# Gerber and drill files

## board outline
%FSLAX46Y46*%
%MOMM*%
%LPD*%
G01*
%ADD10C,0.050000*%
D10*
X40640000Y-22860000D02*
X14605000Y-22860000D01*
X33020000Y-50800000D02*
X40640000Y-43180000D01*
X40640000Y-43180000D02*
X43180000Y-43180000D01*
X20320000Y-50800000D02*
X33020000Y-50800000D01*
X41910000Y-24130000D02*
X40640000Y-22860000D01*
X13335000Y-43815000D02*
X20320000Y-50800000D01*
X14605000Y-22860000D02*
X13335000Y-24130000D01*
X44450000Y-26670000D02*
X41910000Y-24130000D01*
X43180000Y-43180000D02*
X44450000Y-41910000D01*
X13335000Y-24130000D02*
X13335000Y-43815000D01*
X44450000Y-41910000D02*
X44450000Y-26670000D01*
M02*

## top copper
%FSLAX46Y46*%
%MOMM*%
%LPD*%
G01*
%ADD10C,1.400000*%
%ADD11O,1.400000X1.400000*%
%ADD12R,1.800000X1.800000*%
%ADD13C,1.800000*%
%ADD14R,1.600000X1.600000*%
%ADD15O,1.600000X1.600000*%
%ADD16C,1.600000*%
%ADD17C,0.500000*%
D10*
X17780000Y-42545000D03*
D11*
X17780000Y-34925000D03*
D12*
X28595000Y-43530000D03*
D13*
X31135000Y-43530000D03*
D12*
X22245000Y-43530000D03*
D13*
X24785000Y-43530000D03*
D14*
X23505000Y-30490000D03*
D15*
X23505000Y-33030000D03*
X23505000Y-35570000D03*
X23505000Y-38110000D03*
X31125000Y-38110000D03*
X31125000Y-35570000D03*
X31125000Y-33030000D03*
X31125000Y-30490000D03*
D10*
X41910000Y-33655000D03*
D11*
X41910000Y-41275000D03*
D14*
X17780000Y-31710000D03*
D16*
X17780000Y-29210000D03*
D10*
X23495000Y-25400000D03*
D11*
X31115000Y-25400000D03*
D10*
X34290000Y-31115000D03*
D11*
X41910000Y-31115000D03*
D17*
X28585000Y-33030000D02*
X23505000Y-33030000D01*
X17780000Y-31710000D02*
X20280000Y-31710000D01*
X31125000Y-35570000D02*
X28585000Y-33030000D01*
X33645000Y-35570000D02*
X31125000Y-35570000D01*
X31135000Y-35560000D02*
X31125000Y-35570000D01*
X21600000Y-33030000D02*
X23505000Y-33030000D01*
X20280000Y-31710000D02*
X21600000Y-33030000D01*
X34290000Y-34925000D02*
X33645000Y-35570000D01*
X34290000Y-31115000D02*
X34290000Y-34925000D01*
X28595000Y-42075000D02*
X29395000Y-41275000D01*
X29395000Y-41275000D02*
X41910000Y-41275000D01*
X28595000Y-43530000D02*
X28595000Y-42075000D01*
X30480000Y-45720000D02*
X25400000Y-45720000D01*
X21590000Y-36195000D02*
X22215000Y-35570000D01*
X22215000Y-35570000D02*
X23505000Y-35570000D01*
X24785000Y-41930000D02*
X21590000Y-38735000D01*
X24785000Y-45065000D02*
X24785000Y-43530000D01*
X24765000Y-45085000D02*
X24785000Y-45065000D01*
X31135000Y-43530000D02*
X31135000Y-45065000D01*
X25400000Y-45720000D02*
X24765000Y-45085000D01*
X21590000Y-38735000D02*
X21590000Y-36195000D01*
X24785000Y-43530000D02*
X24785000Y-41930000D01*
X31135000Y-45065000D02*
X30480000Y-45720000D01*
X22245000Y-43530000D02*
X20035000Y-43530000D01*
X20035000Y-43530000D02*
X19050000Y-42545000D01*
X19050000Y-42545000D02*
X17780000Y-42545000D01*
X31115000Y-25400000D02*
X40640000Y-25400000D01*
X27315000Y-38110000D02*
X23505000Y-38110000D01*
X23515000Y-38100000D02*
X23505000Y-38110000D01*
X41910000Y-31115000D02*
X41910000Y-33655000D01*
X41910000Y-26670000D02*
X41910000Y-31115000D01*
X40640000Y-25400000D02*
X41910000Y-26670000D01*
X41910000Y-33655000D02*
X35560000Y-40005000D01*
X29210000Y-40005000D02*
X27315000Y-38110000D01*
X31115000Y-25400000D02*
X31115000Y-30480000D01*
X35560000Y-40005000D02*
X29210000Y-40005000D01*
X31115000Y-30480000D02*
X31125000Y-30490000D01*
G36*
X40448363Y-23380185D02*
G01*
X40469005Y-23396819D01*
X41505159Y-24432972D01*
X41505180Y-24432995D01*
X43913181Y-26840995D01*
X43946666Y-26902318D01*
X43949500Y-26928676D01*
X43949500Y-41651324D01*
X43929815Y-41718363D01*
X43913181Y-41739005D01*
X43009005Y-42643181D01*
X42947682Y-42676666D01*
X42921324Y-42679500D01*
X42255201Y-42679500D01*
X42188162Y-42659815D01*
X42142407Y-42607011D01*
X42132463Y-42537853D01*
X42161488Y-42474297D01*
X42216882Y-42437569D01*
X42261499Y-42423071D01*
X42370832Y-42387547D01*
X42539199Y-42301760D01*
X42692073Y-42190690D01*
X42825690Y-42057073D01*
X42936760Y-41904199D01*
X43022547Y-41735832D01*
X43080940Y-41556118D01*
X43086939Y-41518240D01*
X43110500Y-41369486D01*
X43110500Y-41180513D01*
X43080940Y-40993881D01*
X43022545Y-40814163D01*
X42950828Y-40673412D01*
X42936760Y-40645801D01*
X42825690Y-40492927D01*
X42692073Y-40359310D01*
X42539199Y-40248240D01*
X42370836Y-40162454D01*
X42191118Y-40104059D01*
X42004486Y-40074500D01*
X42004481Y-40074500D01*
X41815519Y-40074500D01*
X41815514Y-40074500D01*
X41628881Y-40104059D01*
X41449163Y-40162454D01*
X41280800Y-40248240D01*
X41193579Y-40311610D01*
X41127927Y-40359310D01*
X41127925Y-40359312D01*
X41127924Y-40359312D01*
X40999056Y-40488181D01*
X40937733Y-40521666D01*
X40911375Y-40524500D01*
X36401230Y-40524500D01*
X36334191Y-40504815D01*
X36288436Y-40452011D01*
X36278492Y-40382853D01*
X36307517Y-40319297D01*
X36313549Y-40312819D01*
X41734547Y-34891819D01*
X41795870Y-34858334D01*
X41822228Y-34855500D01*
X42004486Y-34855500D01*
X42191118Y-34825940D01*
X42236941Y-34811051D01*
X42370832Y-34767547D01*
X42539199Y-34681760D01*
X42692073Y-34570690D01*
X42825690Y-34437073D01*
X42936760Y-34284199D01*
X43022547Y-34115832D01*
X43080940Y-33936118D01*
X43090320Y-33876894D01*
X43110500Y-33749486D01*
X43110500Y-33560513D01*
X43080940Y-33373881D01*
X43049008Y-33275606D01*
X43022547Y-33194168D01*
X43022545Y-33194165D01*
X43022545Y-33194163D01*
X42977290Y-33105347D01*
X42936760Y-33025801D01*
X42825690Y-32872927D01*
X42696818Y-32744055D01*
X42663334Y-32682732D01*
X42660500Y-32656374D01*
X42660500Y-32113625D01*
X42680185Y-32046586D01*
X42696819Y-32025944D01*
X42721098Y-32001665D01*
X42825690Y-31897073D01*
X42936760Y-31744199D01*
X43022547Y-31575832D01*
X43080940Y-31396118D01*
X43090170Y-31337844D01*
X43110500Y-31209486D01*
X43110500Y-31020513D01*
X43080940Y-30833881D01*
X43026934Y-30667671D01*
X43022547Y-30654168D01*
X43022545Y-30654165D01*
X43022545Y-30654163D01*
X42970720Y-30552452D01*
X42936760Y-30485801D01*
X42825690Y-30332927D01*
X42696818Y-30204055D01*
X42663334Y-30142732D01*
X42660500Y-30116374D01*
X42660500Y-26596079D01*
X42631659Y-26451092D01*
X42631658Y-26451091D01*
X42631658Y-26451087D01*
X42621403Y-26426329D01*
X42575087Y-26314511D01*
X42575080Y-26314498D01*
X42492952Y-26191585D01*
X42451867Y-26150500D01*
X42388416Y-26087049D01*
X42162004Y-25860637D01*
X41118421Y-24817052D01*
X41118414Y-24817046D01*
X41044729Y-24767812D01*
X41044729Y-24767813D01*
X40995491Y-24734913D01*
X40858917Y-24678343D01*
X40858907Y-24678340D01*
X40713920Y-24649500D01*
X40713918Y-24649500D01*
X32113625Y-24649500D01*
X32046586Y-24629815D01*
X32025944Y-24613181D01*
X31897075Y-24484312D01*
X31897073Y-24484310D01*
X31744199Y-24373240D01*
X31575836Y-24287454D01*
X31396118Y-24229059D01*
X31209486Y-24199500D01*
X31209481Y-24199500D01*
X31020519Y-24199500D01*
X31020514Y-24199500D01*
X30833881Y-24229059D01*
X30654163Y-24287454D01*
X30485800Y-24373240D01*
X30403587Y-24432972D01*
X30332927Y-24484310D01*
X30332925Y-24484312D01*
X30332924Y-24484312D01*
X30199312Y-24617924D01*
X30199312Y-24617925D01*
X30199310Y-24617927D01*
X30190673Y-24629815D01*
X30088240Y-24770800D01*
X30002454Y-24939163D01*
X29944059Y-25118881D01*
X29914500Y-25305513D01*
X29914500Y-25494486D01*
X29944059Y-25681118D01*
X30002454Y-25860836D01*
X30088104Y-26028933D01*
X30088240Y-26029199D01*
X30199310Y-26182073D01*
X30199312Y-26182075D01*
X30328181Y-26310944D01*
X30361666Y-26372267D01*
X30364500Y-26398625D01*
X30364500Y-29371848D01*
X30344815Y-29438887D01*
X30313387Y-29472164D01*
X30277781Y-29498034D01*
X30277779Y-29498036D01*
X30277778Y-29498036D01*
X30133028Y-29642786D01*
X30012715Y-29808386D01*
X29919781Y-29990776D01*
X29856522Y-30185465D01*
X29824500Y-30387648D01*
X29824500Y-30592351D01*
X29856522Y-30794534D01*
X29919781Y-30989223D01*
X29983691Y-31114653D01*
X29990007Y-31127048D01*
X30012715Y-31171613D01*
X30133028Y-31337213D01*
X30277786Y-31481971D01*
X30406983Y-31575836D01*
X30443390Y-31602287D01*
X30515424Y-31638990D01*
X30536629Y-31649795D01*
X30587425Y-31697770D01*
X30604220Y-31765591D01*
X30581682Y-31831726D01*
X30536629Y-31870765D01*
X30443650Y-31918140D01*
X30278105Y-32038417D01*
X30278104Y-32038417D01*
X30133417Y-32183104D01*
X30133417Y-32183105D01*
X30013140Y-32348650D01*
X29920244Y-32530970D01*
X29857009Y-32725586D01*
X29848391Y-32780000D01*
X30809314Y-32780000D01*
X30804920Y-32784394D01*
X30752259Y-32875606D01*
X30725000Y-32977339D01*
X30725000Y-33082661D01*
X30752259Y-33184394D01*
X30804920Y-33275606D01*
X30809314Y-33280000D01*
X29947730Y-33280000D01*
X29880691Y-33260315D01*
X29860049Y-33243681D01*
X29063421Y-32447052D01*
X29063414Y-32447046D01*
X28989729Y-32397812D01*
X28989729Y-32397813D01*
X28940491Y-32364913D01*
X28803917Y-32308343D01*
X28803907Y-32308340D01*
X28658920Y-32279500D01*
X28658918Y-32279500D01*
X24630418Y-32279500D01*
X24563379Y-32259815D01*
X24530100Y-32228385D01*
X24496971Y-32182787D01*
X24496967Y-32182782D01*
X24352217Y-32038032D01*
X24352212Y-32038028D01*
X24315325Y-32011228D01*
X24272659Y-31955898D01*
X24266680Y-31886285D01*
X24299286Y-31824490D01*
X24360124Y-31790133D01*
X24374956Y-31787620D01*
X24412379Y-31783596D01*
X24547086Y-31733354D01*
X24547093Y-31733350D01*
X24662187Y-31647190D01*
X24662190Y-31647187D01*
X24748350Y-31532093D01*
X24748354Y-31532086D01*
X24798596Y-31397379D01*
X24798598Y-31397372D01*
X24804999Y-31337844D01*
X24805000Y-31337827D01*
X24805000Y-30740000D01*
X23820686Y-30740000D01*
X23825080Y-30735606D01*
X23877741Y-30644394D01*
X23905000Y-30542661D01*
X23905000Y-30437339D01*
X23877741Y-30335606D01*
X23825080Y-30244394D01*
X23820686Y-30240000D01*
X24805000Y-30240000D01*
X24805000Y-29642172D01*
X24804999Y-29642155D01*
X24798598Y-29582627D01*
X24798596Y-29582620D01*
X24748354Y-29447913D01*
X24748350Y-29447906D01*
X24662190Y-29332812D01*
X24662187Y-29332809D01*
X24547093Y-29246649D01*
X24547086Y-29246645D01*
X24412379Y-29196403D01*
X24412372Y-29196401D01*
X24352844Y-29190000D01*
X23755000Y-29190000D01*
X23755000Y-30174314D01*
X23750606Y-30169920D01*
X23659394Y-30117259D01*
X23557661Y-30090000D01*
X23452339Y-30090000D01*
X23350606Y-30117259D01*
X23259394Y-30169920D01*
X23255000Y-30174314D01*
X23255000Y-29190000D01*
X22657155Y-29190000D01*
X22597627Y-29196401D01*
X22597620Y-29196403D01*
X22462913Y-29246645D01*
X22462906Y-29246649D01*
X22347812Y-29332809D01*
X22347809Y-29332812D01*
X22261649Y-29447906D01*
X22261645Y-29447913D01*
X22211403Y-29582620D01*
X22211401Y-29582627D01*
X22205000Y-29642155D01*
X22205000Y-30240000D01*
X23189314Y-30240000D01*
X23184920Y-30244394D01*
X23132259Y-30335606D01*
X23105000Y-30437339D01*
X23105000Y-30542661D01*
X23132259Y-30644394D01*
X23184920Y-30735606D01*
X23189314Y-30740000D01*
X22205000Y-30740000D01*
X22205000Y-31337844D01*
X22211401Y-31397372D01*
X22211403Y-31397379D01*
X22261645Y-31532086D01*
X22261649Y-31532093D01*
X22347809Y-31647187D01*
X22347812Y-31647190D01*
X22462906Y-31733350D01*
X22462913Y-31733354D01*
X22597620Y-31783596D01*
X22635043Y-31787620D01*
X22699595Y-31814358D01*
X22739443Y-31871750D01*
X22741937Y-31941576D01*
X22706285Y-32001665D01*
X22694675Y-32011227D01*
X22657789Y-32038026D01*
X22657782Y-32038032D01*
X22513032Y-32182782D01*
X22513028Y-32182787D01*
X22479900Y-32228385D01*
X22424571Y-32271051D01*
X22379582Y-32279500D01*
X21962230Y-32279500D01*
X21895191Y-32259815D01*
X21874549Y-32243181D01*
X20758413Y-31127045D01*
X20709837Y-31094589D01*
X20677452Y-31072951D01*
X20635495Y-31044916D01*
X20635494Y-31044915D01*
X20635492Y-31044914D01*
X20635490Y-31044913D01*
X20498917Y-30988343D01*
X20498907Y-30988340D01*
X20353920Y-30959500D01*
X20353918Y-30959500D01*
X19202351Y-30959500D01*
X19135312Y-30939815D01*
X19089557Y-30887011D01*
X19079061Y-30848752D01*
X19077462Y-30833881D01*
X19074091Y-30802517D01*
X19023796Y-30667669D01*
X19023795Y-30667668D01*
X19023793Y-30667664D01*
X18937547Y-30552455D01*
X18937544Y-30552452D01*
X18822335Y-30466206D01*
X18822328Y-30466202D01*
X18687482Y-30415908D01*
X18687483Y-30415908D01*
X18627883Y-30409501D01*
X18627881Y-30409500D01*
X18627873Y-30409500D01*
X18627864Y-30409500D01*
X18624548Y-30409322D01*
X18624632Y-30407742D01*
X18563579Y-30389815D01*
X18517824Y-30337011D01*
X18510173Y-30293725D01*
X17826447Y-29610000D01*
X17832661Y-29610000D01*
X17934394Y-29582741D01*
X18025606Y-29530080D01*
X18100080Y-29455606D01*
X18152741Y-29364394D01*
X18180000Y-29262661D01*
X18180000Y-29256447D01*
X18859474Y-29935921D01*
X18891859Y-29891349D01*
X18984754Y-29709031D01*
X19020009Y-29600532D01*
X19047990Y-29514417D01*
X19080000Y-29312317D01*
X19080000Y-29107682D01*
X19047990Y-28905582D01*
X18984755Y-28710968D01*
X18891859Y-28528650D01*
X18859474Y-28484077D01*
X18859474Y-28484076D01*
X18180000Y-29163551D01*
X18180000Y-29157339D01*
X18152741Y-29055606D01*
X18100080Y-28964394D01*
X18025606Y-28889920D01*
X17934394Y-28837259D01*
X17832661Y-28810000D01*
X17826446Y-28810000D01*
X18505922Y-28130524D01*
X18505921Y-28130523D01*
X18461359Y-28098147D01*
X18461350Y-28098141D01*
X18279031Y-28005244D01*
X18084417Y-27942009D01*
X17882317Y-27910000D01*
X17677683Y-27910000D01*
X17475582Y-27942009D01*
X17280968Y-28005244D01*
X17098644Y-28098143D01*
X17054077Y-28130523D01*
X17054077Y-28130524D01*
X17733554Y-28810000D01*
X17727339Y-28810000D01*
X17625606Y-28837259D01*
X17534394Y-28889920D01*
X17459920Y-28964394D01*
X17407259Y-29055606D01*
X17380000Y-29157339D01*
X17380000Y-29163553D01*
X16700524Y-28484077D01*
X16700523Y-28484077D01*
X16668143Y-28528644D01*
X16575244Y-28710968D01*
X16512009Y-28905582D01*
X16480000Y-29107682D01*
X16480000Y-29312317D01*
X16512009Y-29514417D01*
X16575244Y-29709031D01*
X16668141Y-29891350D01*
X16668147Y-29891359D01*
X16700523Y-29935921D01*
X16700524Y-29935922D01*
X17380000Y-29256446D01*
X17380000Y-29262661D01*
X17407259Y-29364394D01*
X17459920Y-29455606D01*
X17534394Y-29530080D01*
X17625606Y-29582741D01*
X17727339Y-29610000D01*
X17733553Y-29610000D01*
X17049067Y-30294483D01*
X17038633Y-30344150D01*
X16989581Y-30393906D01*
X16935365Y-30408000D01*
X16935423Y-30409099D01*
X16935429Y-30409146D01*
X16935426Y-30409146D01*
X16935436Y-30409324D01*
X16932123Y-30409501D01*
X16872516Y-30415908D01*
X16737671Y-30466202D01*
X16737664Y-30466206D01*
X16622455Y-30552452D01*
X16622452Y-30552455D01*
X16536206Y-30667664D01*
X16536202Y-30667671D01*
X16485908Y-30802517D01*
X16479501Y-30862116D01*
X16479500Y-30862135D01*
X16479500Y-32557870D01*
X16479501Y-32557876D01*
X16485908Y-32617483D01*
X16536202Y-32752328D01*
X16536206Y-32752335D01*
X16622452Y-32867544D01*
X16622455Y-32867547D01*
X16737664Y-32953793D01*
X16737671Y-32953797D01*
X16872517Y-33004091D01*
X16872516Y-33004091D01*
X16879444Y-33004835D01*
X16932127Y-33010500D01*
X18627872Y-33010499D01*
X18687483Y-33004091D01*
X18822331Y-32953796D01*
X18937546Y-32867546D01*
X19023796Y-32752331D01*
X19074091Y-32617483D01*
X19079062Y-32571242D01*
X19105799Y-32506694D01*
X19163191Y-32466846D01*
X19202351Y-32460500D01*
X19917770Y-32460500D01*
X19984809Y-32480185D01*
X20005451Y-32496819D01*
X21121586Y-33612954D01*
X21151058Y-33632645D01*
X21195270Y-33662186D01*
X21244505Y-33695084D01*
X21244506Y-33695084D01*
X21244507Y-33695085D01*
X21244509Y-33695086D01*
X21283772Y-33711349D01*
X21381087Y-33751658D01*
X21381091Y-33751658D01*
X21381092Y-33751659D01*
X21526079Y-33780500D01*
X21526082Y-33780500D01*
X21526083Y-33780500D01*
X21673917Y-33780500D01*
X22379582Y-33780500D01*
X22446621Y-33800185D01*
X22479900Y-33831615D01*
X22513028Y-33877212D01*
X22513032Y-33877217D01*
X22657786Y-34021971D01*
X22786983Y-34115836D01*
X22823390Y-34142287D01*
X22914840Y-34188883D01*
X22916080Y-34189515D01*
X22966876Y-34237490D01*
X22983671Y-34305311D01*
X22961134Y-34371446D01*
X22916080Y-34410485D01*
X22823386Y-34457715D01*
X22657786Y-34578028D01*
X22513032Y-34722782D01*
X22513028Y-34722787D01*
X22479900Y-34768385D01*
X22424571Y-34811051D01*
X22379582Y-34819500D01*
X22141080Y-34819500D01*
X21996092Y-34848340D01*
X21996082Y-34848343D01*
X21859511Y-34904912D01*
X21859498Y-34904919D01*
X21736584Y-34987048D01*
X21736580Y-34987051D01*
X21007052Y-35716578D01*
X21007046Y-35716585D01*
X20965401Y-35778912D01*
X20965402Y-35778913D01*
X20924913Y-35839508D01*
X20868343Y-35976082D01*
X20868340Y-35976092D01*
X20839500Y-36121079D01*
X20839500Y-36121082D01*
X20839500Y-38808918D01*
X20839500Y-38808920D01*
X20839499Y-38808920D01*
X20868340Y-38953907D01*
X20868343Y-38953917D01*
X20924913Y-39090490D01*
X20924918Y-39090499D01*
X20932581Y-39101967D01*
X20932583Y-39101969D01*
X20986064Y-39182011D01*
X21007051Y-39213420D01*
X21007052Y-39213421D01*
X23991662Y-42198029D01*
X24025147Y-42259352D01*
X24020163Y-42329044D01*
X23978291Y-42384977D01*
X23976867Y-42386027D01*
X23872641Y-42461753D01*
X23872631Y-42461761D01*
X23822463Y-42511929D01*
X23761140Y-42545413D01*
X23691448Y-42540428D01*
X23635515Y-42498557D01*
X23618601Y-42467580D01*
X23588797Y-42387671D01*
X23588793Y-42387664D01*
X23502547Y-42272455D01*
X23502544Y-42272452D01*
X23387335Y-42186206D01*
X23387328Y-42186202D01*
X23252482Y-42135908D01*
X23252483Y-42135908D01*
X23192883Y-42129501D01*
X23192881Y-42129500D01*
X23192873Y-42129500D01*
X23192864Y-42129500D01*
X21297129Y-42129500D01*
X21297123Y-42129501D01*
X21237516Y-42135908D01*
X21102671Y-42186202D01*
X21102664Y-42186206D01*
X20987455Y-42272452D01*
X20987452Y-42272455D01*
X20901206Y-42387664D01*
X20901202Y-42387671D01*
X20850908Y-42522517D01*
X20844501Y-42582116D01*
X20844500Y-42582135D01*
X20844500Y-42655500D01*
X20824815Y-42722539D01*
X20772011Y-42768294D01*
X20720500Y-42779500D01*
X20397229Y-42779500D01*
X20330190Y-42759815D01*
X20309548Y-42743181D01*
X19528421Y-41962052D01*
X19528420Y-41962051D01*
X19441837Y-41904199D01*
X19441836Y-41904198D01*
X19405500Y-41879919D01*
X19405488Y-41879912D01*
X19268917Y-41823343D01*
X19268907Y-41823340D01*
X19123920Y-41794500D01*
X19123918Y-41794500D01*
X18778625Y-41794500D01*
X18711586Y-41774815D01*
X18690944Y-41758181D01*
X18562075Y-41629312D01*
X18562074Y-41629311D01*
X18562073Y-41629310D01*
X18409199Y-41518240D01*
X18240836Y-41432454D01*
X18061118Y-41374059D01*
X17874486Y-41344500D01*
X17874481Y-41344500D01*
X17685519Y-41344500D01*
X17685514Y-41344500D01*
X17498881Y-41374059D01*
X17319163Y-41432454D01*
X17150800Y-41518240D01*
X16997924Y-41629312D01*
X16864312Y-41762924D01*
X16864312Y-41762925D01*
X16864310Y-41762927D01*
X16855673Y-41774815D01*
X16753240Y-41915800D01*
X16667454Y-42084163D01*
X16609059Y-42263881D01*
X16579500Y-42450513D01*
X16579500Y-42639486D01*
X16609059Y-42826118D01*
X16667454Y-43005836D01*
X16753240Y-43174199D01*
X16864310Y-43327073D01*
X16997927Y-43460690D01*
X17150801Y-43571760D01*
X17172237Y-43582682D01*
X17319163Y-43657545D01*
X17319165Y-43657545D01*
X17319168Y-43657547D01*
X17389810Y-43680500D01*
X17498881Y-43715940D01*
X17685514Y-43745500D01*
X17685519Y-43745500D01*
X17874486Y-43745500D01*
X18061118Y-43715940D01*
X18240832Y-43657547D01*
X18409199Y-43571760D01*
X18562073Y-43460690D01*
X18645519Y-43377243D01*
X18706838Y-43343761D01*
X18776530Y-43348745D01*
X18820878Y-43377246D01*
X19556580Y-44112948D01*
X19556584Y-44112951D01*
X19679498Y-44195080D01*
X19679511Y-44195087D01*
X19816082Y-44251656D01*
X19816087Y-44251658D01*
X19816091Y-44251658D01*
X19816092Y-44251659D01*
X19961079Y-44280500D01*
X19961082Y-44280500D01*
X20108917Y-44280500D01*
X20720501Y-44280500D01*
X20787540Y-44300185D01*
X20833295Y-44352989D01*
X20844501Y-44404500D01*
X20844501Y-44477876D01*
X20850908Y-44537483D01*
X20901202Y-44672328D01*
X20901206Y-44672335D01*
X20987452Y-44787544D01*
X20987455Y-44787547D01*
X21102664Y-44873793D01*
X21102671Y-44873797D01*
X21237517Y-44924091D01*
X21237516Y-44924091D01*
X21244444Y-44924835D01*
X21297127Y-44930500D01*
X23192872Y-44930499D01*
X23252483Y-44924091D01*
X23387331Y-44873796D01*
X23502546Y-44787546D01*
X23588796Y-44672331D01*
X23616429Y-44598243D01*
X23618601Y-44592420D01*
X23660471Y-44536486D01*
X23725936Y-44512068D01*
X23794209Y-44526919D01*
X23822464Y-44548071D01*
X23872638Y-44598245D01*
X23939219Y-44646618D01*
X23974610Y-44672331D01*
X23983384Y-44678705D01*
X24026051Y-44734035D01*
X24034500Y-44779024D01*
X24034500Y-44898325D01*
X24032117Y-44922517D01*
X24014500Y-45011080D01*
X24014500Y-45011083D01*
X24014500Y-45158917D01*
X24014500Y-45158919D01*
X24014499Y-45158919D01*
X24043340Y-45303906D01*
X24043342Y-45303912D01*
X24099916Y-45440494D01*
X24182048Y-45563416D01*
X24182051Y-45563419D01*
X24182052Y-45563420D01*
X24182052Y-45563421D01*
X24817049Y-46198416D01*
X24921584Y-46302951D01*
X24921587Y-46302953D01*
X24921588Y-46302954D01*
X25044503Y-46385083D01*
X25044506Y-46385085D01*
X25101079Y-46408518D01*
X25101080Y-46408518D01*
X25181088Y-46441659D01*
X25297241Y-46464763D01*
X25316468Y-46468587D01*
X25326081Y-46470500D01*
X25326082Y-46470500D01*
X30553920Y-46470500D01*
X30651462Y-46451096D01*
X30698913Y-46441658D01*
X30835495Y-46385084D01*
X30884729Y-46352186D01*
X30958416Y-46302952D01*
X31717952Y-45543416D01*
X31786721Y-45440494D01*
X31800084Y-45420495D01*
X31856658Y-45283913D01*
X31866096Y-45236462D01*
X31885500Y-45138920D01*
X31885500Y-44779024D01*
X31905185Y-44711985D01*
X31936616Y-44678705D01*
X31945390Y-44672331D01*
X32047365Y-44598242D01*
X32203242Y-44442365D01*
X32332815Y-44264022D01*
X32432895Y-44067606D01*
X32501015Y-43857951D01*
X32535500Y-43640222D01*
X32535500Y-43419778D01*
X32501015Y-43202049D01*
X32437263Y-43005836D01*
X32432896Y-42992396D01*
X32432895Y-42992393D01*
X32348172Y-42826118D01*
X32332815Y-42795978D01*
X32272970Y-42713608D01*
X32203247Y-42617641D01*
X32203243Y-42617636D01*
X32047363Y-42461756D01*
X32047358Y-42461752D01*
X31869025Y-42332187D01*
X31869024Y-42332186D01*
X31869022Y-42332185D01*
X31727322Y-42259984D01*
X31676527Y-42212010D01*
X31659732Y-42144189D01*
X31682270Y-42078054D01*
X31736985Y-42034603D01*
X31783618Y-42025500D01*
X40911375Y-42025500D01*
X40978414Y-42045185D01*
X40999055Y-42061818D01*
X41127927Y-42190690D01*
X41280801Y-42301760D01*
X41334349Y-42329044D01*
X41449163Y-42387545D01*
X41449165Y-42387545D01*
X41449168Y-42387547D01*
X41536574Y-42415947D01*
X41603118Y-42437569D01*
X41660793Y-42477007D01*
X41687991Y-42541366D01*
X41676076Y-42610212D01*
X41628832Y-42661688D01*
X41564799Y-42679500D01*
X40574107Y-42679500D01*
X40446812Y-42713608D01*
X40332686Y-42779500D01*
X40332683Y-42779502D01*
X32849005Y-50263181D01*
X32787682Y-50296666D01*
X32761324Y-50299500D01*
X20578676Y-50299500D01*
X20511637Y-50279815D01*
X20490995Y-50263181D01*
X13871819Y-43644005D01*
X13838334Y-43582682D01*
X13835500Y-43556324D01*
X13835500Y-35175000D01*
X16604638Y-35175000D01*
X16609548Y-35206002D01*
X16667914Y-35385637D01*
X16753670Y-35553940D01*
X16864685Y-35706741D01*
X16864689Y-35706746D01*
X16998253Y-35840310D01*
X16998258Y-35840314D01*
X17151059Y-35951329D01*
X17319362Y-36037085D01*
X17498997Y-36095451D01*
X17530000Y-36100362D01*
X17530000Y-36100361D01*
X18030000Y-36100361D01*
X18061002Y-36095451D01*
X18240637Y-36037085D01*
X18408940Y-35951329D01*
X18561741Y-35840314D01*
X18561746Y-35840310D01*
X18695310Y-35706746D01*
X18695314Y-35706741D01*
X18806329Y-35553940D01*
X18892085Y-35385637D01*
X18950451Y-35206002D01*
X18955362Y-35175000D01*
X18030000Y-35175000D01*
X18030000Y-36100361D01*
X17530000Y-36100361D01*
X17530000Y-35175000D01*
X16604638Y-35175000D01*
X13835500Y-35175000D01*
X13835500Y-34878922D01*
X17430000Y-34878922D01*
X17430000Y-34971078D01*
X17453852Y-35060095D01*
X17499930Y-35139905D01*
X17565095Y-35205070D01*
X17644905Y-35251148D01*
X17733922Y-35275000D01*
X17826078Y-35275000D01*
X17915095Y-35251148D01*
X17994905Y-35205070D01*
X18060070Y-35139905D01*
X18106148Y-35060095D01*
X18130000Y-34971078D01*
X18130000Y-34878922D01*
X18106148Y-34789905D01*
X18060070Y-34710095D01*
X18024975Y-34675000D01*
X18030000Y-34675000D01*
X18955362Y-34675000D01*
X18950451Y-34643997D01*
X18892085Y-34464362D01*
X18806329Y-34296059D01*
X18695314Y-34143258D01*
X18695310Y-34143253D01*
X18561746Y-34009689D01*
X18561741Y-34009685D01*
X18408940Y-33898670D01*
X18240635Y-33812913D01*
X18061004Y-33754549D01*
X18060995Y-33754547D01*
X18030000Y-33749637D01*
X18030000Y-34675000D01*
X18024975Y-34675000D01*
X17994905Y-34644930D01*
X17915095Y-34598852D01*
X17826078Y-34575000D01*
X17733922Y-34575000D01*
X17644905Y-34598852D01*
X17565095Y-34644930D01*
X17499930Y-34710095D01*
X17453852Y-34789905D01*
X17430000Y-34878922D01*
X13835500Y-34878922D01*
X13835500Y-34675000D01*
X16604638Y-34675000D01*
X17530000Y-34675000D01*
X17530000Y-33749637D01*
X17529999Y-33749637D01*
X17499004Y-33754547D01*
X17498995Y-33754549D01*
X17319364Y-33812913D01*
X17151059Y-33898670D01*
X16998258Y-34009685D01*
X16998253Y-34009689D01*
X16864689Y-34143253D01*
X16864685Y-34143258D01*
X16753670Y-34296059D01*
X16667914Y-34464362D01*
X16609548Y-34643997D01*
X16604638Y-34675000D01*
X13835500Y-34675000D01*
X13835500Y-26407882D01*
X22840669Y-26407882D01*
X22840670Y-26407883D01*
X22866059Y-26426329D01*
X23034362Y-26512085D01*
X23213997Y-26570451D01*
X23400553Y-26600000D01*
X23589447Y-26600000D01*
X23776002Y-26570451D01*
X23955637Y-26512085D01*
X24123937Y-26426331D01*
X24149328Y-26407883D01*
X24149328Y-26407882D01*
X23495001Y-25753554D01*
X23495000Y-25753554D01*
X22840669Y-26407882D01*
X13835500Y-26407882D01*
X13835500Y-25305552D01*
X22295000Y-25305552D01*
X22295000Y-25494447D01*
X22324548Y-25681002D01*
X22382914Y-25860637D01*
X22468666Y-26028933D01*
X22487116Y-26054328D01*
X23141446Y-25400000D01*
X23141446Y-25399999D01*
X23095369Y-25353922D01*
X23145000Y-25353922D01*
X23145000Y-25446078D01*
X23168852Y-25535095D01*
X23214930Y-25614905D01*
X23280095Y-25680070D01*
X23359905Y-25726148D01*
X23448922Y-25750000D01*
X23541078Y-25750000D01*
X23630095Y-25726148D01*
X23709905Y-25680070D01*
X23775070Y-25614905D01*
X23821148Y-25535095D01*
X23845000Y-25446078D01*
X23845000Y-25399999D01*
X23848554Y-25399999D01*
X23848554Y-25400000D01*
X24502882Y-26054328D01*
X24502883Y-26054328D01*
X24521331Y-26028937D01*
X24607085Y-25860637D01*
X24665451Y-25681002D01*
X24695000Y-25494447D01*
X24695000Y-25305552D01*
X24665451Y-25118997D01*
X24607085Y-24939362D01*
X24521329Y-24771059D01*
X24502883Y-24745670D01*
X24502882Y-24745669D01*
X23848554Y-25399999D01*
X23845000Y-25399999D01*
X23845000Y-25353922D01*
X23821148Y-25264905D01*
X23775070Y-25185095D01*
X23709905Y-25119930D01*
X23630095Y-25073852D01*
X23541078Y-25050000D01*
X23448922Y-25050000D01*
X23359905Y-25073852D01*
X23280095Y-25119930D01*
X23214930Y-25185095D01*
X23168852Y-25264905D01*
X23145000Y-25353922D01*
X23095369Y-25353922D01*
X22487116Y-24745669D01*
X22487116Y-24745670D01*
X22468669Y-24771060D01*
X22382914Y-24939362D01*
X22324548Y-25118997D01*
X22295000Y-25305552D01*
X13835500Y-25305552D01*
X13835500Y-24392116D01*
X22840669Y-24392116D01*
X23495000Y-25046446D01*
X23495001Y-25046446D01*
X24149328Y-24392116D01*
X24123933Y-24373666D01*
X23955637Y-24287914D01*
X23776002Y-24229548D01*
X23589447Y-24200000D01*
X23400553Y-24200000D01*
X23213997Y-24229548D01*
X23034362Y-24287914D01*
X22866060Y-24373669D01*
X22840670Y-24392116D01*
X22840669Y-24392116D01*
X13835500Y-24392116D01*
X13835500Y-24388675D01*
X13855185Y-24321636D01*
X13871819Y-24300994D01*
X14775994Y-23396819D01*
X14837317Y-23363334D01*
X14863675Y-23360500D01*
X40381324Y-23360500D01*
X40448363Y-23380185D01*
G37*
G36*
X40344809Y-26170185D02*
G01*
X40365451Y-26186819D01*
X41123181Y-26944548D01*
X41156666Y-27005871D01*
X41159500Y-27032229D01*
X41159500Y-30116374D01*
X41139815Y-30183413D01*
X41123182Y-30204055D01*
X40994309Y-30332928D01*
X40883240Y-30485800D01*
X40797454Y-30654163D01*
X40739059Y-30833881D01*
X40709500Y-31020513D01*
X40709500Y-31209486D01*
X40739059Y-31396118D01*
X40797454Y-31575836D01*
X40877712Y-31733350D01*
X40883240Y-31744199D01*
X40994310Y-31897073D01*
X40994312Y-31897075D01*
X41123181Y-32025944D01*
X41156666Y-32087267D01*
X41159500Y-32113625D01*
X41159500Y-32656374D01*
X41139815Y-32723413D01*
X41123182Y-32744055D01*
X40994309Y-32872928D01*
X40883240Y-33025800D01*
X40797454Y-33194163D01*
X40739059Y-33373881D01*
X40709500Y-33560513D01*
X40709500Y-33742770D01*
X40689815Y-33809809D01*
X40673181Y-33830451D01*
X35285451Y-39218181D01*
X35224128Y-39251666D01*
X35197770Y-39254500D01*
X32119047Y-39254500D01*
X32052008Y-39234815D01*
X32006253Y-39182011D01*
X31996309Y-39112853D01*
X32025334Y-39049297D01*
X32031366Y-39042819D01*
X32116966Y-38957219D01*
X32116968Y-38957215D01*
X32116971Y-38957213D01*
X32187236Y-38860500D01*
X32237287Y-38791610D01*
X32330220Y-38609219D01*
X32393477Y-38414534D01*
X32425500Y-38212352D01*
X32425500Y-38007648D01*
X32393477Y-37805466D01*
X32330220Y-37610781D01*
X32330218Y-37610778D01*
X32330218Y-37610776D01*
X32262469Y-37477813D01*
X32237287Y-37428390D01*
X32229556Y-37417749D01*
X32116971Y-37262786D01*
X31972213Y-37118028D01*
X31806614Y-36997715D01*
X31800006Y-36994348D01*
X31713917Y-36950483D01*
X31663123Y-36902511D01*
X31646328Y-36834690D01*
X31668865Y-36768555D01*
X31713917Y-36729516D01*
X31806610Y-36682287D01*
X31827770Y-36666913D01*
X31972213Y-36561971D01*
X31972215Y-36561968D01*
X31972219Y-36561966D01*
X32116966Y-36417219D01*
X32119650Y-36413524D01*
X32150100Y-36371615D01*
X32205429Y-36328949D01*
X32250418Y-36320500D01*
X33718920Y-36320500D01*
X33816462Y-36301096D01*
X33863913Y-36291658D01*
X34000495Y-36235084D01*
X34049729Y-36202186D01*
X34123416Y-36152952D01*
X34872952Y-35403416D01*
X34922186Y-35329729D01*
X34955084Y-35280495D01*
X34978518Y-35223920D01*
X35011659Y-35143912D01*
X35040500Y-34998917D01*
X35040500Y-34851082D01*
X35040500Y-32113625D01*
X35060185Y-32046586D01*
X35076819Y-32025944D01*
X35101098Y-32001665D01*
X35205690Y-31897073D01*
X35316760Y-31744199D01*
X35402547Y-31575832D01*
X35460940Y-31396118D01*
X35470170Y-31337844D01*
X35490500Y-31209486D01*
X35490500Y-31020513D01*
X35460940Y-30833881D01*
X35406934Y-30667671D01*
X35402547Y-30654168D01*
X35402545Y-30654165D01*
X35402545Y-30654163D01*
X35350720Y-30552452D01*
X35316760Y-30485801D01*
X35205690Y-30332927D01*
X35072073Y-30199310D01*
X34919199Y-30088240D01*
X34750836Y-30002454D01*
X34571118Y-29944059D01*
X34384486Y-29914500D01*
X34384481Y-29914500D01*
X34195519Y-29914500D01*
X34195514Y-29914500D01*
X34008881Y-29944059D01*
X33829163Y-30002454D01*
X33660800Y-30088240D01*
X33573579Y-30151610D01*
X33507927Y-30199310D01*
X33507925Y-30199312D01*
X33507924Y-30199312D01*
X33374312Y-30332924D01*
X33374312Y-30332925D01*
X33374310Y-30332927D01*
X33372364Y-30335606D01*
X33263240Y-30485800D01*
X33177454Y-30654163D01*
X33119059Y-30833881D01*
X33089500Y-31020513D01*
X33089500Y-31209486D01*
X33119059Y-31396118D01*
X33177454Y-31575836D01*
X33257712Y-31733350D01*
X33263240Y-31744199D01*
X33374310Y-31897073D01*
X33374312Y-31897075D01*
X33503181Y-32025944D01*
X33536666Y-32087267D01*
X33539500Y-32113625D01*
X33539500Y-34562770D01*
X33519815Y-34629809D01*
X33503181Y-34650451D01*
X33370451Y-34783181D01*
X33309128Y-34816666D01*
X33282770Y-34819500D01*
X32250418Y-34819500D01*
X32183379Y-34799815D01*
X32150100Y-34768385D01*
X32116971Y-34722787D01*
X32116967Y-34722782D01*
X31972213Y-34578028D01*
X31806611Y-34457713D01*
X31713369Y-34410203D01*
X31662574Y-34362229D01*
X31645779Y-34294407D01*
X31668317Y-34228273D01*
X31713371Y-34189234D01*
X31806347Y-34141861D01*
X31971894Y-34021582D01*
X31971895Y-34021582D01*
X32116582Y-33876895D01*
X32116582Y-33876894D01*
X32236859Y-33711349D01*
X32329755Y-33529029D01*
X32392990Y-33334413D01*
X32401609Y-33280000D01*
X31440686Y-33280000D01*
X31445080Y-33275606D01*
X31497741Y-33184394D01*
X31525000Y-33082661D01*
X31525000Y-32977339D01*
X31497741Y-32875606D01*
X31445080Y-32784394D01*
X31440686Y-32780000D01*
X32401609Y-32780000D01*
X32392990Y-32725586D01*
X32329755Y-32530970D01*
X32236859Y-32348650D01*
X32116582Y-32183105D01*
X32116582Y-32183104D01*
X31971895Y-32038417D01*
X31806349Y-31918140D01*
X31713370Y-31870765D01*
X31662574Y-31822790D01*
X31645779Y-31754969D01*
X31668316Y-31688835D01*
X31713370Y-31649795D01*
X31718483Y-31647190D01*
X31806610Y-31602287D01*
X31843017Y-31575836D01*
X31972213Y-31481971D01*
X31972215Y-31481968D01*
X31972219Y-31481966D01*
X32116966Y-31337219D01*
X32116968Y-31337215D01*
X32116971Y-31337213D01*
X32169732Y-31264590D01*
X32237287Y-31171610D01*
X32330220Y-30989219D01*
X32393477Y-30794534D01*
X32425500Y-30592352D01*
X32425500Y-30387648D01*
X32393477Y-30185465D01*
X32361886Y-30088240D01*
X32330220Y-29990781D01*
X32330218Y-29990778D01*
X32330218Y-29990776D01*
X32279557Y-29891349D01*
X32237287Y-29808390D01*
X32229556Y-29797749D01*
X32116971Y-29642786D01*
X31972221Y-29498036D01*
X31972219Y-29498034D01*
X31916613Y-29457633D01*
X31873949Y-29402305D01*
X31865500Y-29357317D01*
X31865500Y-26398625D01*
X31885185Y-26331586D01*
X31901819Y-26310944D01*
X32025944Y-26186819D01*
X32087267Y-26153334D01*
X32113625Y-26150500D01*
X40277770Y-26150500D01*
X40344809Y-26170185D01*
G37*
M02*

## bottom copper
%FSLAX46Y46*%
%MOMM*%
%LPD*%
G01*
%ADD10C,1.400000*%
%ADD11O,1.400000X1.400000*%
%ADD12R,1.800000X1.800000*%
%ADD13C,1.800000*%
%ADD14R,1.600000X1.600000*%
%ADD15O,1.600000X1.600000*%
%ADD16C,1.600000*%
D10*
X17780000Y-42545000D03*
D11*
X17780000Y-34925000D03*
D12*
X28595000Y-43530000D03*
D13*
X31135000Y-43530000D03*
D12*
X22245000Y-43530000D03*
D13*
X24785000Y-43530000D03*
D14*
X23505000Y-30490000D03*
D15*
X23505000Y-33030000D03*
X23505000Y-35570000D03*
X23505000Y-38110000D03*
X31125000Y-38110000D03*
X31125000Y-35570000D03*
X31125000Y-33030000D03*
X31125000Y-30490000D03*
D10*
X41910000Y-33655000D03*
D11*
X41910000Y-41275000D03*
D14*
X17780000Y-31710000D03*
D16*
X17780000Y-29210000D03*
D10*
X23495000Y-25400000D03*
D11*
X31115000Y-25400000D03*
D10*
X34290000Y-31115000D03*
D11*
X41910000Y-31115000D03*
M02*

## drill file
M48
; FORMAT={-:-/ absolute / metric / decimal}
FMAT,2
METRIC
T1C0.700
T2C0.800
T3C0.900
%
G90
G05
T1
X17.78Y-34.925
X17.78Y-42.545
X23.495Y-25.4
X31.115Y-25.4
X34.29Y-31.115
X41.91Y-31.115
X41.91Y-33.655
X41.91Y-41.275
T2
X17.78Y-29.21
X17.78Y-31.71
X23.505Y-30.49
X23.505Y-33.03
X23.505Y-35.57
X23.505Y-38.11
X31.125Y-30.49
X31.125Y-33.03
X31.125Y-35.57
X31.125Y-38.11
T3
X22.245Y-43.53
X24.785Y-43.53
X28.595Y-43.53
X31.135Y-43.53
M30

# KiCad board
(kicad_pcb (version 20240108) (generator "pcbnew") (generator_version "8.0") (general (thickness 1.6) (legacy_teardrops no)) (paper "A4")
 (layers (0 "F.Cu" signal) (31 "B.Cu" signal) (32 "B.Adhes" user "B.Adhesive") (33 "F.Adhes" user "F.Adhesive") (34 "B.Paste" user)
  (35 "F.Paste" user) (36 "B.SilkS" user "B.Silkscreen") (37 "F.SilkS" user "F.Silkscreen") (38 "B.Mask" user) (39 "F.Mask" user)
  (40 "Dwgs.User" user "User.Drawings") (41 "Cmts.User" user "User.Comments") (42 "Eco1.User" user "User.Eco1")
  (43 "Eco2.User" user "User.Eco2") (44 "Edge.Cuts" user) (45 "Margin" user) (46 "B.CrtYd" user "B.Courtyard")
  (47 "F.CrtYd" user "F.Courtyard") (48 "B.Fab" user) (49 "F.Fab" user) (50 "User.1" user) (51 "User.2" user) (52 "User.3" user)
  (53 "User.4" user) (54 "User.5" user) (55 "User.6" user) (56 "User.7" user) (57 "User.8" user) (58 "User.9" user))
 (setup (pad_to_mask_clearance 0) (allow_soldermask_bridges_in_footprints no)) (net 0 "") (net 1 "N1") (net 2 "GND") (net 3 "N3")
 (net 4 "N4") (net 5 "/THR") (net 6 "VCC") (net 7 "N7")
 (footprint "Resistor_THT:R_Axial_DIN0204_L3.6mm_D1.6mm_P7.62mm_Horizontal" (layer "F.Cu") (at 17.78 42.545 90)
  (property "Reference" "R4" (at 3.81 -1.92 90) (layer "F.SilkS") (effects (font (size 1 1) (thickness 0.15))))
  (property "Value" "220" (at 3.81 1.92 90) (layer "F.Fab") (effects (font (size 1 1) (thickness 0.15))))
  (pad "1" thru_hole circle (at 0 0 90) (size 1.4 1.4) (drill 0.7) (layers "*.Cu" "*.Mask") (remove_unused_layers no) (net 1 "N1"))
  (pad "2" thru_hole oval (at 7.62 0 90) (size 1.4 1.4) (drill 0.7) (layers "*.Cu" "*.Mask") (remove_unused_layers no) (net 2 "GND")))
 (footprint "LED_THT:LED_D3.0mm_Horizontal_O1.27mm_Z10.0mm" (layer "F.Cu") (at 28.595 43.53)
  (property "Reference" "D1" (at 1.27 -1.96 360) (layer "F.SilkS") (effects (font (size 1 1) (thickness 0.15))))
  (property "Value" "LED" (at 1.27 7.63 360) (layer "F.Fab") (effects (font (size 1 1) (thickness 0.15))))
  (pad "1" thru_hole rect (at 0 0) (size 1.8 1.8) (drill 0.9) (layers "*.Cu" "*.Mask") (remove_unused_layers no) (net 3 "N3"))
  (pad "2" thru_hole circle (at 2.54 0) (size 1.8 1.8) (drill 0.9) (layers "*.Cu" "*.Mask") (remove_unused_layers no) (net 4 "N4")))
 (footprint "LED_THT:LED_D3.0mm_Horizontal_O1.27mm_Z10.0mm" (layer "F.Cu") (at 22.245 43.53)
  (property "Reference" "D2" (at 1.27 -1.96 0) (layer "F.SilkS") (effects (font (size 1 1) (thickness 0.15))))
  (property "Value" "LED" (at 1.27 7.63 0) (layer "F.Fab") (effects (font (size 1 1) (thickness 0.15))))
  (pad "1" thru_hole rect (at 0 0) (size 1.8 1.8) (drill 0.9) (layers "*.Cu" "*.Mask") (remove_unused_layers no) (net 1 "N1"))
  (pad "2" thru_hole circle (at 2.54 0) (size 1.8 1.8) (drill 0.9) (layers "*.Cu" "*.Mask") (remove_unused_layers no) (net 4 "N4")))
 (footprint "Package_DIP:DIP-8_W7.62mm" (layer "F.Cu") (at 23.505 30.49)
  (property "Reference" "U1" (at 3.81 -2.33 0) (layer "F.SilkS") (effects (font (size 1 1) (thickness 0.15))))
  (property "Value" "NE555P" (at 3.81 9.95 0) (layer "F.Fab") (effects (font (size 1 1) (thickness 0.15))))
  (pad "1" thru_hole rect (at 0 0) (size 1.6 1.6) (drill 0.8) (layers "*.Cu" "*.Mask") (remove_unused_layers no) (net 2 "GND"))
  (pad "2" thru_hole oval (at 0 2.54) (size 1.6 1.6) (drill 0.8) (layers "*.Cu" "*.Mask") (remove_unused_layers no) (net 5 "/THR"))
  (pad "3" thru_hole oval (at 0 5.08) (size 1.6 1.6) (drill 0.8) (layers "*.Cu" "*.Mask") (remove_unused_layers no) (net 4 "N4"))
  (pad "4" thru_hole oval (at 0 7.62) (size 1.6 1.6) (drill 0.8) (layers "*.Cu" "*.Mask") (remove_unused_layers no) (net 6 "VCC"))
  (pad "5" thru_hole oval (at 7.62 7.62) (size 1.6 1.6) (drill 0.8) (layers "*.Cu" "*.Mask") (remove_unused_layers no) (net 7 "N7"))
  (pad "6" thru_hole oval (at 7.62 5.08) (size 1.6 1.6) (drill 0.8) (layers "*.Cu" "*.Mask") (remove_unused_layers no) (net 5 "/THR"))
  (pad "7" thru_hole oval (at 7.62 2.54) (size 1.6 1.6) (drill 0.8) (layers "*.Cu" "*.Mask") (remove_unused_layers no) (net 2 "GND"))
  (pad "8" thru_hole oval (at 7.62 0) (size 1.6 1.6) (drill 0.8) (layers "*.Cu" "*.Mask") (remove_unused_layers no) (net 6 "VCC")))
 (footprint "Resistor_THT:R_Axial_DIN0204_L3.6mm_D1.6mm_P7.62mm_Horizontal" (layer "F.Cu") (at 41.91 33.655 -90)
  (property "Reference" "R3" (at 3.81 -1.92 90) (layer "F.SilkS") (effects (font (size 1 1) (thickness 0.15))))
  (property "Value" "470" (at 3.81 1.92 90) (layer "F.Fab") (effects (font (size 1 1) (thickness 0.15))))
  (pad "1" thru_hole circle (at 0 0 270) (size 1.4 1.4) (drill 0.7) (layers "*.Cu" "*.Mask") (remove_unused_layers no) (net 6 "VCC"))
  (pad "2" thru_hole oval (at 7.62 0 270) (size 1.4 1.4) (drill 0.7) (layers "*.Cu" "*.Mask") (remove_unused_layers no) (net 3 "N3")))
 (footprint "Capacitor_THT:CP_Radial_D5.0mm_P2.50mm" (layer "F.Cu") (at 17.78 31.71 90)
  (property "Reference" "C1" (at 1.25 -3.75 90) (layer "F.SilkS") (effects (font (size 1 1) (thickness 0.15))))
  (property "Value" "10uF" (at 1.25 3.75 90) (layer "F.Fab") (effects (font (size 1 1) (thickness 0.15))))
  (pad "1" thru_hole rect (at 0 0 90) (size 1.6 1.6) (drill 0.8) (layers "*.Cu" "*.Mask") (remove_unused_layers no) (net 5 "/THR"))
  (pad "2" thru_hole circle (at 2.5 0 90) (size 1.6 1.6) (drill 0.8) (layers "*.Cu" "*.Mask") (remove_unused_layers no) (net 2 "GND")))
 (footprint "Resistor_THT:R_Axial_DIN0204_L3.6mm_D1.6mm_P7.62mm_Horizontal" (layer "F.Cu") (at 23.495 25.4)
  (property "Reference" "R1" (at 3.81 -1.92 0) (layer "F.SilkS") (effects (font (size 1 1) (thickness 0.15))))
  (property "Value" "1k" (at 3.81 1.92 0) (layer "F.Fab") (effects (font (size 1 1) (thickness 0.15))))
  (pad "1" thru_hole circle (at 0 0) (size 1.4 1.4) (drill 0.7) (layers "*.Cu" "*.Mask") (remove_unused_layers no) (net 2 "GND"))
  (pad "2" thru_hole oval (at 7.62 0) (size 1.4 1.4) (drill 0.7) (layers "*.Cu" "*.Mask") (remove_unused_layers no) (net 6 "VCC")))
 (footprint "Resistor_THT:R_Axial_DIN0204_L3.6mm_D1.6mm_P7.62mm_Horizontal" (layer "F.Cu") (at 34.29 31.115)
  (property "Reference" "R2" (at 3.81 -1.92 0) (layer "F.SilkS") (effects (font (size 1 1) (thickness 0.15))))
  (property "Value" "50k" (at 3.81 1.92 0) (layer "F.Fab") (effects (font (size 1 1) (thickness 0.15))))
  (pad "1" thru_hole circle (at 0 0) (size 1.4 1.4) (drill 0.7) (layers "*.Cu" "*.Mask") (remove_unused_layers no) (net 5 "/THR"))
  (pad "2" thru_hole oval (at 7.62 0) (size 1.4 1.4) (drill 0.7) (layers "*.Cu" "*.Mask") (remove_unused_layers no) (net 6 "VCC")))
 (gr_line (start 40.64 22.86) (end 14.605 22.86) (stroke (width 0.05) (type default)) (layer "Edge.Cuts"))
 (gr_line (start 33.02 50.8) (end 40.64 43.18) (stroke (width 0.05) (type default)) (layer "Edge.Cuts"))
 (gr_line (start 40.64 43.18) (end 43.18 43.18) (stroke (width 0.05) (type default)) (layer "Edge.Cuts"))
 (gr_line (start 20.32 50.8) (end 33.02 50.8) (stroke (width 0.05) (type default)) (layer "Edge.Cuts"))
 (gr_line (start 41.91 24.13) (end 40.64 22.86) (stroke (width 0.05) (type default)) (layer "Edge.Cuts"))
 (gr_line (start 13.335 43.815) (end 20.32 50.8) (stroke (width 0.05) (type default)) (layer "Edge.Cuts"))
 (gr_line (start 14.605 22.86) (end 13.335 24.13) (stroke (width 0.05) (type default)) (layer "Edge.Cuts"))
 (gr_line (start 44.45 26.67) (end 41.91 24.13) (stroke (width 0.05) (type default)) (layer "Edge.Cuts"))
 (gr_line (start 43.18 43.18) (end 44.45 41.91) (stroke (width 0.05) (type default)) (layer "Edge.Cuts"))
 (gr_line (start 13.335 24.13) (end 13.335 43.815) (stroke (width 0.05) (type default)) (layer "Edge.Cuts"))
 (gr_line (start 44.45 41.91) (end 44.45 26.67) (stroke (width 0.05) (type default)) (layer "Edge.Cuts"))
 (segment (start 28.585 33.03) (end 23.505 33.03) (width 0.5) (layer "F.Cu") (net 5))
 (segment (start 17.78 31.71) (end 20.28 31.71) (width 0.5) (layer "F.Cu") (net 5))
 (segment (start 31.125 35.57) (end 28.585 33.03) (width 0.5) (layer "F.Cu") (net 5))
 (segment (start 33.645 35.57) (end 31.125 35.57) (width 0.5) (layer "F.Cu") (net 5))
 (segment (start 31.135 35.56) (end 31.125 35.57) (width 0.5) (layer "F.Cu") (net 5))
 (segment (start 21.6 33.03) (end 23.505 33.03) (width 0.5) (layer "F.Cu") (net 5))
 (segment (start 20.28 31.71) (end 21.6 33.03) (width 0.5) (layer "F.Cu") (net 5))
 (segment (start 34.29 34.925) (end 33.645 35.57) (width 0.5) (layer "F.Cu") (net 5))
 (segment (start 34.29 31.115) (end 34.29 34.925) (width 0.5) (layer "F.Cu") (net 5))
 (segment (start 28.595 42.075) (end 29.395 41.275) (width 0.5) (layer "F.Cu") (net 3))
 (segment (start 29.395 41.275) (end 41.91 41.275) (width 0.5) (layer "F.Cu") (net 3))
 (segment (start 28.595 43.53) (end 28.595 42.075) (width 0.5) (layer "F.Cu") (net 3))
 (segment (start 30.48 45.72) (end 25.4 45.72) (width 0.5) (layer "F.Cu") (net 4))
 (segment (start 21.59 36.195) (end 22.215 35.57) (width 0.5) (layer "F.Cu") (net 4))
 (segment (start 22.215 35.57) (end 23.505 35.57) (width 0.5) (layer "F.Cu") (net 4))
 (segment (start 24.785 41.93) (end 21.59 38.735) (width 0.5) (layer "F.Cu") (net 4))
 (segment (start 24.785 45.065) (end 24.785 43.53) (width 0.5) (layer "F.Cu") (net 4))
 (segment (start 24.765 45.085) (end 24.785 45.065) (width 0.5) (layer "F.Cu") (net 4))
 (segment (start 31.135 43.53) (end 31.135 45.065) (width 0.5) (layer "F.Cu") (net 4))
 (segment (start 25.4 45.72) (end 24.765 45.085) (width 0.5) (layer "F.Cu") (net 4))
 (segment (start 21.59 38.735) (end 21.59 36.195) (width 0.5) (layer "F.Cu") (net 4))
 (segment (start 24.785 43.53) (end 24.785 41.93) (width 0.5) (layer "F.Cu") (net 4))
 (segment (start 31.135 45.065) (end 30.48 45.72) (width 0.5) (layer "F.Cu") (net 4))
 (segment (start 22.245 43.53) (end 20.035 43.53) (width 0.5) (layer "F.Cu") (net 1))
 (segment (start 20.035 43.53) (end 19.05 42.545) (width 0.5) (layer "F.Cu") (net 1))
 (segment (start 19.05 42.545) (end 17.78 42.545) (width 0.5) (layer "F.Cu") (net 1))
 (segment (start 31.115 25.4) (end 40.64 25.4) (width 0.5) (layer "F.Cu") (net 6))
 (segment (start 27.315 38.11) (end 23.505 38.11) (width 0.5) (layer "F.Cu") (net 6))
 (segment (start 23.515 38.1) (end 23.505 38.11) (width 0.5) (layer "F.Cu") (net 6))
 (segment (start 41.91 31.115) (end 41.91 33.655) (width 0.5) (layer "F.Cu") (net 6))
 (segment (start 41.91 26.67) (end 41.91 31.115) (width 0.5) (layer "F.Cu") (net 6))
 (segment (start 40.64 25.4) (end 41.91 26.67) (width 0.5) (layer "F.Cu") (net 6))
 (segment (start 41.91 33.655) (end 35.56 40.005) (width 0.5) (layer "F.Cu") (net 6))
 (segment (start 29.21 40.005) (end 27.315 38.11) (width 0.5) (layer "F.Cu") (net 6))
 (segment (start 31.115 25.4) (end 31.115 30.48) (width 0.5) (layer "F.Cu") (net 6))
 (segment (start 35.56 40.005) (end 29.21 40.005) (width 0.5) (layer "F.Cu") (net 6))
 (segment (start 31.115 30.48) (end 31.125 30.49) (width 0.5) (layer "F.Cu") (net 6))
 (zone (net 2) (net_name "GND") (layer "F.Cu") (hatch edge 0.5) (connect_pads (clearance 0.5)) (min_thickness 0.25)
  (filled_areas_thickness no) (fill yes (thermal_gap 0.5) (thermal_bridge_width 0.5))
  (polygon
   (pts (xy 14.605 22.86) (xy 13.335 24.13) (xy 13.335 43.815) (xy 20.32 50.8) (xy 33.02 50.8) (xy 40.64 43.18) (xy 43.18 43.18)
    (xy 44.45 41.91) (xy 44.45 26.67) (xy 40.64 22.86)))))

